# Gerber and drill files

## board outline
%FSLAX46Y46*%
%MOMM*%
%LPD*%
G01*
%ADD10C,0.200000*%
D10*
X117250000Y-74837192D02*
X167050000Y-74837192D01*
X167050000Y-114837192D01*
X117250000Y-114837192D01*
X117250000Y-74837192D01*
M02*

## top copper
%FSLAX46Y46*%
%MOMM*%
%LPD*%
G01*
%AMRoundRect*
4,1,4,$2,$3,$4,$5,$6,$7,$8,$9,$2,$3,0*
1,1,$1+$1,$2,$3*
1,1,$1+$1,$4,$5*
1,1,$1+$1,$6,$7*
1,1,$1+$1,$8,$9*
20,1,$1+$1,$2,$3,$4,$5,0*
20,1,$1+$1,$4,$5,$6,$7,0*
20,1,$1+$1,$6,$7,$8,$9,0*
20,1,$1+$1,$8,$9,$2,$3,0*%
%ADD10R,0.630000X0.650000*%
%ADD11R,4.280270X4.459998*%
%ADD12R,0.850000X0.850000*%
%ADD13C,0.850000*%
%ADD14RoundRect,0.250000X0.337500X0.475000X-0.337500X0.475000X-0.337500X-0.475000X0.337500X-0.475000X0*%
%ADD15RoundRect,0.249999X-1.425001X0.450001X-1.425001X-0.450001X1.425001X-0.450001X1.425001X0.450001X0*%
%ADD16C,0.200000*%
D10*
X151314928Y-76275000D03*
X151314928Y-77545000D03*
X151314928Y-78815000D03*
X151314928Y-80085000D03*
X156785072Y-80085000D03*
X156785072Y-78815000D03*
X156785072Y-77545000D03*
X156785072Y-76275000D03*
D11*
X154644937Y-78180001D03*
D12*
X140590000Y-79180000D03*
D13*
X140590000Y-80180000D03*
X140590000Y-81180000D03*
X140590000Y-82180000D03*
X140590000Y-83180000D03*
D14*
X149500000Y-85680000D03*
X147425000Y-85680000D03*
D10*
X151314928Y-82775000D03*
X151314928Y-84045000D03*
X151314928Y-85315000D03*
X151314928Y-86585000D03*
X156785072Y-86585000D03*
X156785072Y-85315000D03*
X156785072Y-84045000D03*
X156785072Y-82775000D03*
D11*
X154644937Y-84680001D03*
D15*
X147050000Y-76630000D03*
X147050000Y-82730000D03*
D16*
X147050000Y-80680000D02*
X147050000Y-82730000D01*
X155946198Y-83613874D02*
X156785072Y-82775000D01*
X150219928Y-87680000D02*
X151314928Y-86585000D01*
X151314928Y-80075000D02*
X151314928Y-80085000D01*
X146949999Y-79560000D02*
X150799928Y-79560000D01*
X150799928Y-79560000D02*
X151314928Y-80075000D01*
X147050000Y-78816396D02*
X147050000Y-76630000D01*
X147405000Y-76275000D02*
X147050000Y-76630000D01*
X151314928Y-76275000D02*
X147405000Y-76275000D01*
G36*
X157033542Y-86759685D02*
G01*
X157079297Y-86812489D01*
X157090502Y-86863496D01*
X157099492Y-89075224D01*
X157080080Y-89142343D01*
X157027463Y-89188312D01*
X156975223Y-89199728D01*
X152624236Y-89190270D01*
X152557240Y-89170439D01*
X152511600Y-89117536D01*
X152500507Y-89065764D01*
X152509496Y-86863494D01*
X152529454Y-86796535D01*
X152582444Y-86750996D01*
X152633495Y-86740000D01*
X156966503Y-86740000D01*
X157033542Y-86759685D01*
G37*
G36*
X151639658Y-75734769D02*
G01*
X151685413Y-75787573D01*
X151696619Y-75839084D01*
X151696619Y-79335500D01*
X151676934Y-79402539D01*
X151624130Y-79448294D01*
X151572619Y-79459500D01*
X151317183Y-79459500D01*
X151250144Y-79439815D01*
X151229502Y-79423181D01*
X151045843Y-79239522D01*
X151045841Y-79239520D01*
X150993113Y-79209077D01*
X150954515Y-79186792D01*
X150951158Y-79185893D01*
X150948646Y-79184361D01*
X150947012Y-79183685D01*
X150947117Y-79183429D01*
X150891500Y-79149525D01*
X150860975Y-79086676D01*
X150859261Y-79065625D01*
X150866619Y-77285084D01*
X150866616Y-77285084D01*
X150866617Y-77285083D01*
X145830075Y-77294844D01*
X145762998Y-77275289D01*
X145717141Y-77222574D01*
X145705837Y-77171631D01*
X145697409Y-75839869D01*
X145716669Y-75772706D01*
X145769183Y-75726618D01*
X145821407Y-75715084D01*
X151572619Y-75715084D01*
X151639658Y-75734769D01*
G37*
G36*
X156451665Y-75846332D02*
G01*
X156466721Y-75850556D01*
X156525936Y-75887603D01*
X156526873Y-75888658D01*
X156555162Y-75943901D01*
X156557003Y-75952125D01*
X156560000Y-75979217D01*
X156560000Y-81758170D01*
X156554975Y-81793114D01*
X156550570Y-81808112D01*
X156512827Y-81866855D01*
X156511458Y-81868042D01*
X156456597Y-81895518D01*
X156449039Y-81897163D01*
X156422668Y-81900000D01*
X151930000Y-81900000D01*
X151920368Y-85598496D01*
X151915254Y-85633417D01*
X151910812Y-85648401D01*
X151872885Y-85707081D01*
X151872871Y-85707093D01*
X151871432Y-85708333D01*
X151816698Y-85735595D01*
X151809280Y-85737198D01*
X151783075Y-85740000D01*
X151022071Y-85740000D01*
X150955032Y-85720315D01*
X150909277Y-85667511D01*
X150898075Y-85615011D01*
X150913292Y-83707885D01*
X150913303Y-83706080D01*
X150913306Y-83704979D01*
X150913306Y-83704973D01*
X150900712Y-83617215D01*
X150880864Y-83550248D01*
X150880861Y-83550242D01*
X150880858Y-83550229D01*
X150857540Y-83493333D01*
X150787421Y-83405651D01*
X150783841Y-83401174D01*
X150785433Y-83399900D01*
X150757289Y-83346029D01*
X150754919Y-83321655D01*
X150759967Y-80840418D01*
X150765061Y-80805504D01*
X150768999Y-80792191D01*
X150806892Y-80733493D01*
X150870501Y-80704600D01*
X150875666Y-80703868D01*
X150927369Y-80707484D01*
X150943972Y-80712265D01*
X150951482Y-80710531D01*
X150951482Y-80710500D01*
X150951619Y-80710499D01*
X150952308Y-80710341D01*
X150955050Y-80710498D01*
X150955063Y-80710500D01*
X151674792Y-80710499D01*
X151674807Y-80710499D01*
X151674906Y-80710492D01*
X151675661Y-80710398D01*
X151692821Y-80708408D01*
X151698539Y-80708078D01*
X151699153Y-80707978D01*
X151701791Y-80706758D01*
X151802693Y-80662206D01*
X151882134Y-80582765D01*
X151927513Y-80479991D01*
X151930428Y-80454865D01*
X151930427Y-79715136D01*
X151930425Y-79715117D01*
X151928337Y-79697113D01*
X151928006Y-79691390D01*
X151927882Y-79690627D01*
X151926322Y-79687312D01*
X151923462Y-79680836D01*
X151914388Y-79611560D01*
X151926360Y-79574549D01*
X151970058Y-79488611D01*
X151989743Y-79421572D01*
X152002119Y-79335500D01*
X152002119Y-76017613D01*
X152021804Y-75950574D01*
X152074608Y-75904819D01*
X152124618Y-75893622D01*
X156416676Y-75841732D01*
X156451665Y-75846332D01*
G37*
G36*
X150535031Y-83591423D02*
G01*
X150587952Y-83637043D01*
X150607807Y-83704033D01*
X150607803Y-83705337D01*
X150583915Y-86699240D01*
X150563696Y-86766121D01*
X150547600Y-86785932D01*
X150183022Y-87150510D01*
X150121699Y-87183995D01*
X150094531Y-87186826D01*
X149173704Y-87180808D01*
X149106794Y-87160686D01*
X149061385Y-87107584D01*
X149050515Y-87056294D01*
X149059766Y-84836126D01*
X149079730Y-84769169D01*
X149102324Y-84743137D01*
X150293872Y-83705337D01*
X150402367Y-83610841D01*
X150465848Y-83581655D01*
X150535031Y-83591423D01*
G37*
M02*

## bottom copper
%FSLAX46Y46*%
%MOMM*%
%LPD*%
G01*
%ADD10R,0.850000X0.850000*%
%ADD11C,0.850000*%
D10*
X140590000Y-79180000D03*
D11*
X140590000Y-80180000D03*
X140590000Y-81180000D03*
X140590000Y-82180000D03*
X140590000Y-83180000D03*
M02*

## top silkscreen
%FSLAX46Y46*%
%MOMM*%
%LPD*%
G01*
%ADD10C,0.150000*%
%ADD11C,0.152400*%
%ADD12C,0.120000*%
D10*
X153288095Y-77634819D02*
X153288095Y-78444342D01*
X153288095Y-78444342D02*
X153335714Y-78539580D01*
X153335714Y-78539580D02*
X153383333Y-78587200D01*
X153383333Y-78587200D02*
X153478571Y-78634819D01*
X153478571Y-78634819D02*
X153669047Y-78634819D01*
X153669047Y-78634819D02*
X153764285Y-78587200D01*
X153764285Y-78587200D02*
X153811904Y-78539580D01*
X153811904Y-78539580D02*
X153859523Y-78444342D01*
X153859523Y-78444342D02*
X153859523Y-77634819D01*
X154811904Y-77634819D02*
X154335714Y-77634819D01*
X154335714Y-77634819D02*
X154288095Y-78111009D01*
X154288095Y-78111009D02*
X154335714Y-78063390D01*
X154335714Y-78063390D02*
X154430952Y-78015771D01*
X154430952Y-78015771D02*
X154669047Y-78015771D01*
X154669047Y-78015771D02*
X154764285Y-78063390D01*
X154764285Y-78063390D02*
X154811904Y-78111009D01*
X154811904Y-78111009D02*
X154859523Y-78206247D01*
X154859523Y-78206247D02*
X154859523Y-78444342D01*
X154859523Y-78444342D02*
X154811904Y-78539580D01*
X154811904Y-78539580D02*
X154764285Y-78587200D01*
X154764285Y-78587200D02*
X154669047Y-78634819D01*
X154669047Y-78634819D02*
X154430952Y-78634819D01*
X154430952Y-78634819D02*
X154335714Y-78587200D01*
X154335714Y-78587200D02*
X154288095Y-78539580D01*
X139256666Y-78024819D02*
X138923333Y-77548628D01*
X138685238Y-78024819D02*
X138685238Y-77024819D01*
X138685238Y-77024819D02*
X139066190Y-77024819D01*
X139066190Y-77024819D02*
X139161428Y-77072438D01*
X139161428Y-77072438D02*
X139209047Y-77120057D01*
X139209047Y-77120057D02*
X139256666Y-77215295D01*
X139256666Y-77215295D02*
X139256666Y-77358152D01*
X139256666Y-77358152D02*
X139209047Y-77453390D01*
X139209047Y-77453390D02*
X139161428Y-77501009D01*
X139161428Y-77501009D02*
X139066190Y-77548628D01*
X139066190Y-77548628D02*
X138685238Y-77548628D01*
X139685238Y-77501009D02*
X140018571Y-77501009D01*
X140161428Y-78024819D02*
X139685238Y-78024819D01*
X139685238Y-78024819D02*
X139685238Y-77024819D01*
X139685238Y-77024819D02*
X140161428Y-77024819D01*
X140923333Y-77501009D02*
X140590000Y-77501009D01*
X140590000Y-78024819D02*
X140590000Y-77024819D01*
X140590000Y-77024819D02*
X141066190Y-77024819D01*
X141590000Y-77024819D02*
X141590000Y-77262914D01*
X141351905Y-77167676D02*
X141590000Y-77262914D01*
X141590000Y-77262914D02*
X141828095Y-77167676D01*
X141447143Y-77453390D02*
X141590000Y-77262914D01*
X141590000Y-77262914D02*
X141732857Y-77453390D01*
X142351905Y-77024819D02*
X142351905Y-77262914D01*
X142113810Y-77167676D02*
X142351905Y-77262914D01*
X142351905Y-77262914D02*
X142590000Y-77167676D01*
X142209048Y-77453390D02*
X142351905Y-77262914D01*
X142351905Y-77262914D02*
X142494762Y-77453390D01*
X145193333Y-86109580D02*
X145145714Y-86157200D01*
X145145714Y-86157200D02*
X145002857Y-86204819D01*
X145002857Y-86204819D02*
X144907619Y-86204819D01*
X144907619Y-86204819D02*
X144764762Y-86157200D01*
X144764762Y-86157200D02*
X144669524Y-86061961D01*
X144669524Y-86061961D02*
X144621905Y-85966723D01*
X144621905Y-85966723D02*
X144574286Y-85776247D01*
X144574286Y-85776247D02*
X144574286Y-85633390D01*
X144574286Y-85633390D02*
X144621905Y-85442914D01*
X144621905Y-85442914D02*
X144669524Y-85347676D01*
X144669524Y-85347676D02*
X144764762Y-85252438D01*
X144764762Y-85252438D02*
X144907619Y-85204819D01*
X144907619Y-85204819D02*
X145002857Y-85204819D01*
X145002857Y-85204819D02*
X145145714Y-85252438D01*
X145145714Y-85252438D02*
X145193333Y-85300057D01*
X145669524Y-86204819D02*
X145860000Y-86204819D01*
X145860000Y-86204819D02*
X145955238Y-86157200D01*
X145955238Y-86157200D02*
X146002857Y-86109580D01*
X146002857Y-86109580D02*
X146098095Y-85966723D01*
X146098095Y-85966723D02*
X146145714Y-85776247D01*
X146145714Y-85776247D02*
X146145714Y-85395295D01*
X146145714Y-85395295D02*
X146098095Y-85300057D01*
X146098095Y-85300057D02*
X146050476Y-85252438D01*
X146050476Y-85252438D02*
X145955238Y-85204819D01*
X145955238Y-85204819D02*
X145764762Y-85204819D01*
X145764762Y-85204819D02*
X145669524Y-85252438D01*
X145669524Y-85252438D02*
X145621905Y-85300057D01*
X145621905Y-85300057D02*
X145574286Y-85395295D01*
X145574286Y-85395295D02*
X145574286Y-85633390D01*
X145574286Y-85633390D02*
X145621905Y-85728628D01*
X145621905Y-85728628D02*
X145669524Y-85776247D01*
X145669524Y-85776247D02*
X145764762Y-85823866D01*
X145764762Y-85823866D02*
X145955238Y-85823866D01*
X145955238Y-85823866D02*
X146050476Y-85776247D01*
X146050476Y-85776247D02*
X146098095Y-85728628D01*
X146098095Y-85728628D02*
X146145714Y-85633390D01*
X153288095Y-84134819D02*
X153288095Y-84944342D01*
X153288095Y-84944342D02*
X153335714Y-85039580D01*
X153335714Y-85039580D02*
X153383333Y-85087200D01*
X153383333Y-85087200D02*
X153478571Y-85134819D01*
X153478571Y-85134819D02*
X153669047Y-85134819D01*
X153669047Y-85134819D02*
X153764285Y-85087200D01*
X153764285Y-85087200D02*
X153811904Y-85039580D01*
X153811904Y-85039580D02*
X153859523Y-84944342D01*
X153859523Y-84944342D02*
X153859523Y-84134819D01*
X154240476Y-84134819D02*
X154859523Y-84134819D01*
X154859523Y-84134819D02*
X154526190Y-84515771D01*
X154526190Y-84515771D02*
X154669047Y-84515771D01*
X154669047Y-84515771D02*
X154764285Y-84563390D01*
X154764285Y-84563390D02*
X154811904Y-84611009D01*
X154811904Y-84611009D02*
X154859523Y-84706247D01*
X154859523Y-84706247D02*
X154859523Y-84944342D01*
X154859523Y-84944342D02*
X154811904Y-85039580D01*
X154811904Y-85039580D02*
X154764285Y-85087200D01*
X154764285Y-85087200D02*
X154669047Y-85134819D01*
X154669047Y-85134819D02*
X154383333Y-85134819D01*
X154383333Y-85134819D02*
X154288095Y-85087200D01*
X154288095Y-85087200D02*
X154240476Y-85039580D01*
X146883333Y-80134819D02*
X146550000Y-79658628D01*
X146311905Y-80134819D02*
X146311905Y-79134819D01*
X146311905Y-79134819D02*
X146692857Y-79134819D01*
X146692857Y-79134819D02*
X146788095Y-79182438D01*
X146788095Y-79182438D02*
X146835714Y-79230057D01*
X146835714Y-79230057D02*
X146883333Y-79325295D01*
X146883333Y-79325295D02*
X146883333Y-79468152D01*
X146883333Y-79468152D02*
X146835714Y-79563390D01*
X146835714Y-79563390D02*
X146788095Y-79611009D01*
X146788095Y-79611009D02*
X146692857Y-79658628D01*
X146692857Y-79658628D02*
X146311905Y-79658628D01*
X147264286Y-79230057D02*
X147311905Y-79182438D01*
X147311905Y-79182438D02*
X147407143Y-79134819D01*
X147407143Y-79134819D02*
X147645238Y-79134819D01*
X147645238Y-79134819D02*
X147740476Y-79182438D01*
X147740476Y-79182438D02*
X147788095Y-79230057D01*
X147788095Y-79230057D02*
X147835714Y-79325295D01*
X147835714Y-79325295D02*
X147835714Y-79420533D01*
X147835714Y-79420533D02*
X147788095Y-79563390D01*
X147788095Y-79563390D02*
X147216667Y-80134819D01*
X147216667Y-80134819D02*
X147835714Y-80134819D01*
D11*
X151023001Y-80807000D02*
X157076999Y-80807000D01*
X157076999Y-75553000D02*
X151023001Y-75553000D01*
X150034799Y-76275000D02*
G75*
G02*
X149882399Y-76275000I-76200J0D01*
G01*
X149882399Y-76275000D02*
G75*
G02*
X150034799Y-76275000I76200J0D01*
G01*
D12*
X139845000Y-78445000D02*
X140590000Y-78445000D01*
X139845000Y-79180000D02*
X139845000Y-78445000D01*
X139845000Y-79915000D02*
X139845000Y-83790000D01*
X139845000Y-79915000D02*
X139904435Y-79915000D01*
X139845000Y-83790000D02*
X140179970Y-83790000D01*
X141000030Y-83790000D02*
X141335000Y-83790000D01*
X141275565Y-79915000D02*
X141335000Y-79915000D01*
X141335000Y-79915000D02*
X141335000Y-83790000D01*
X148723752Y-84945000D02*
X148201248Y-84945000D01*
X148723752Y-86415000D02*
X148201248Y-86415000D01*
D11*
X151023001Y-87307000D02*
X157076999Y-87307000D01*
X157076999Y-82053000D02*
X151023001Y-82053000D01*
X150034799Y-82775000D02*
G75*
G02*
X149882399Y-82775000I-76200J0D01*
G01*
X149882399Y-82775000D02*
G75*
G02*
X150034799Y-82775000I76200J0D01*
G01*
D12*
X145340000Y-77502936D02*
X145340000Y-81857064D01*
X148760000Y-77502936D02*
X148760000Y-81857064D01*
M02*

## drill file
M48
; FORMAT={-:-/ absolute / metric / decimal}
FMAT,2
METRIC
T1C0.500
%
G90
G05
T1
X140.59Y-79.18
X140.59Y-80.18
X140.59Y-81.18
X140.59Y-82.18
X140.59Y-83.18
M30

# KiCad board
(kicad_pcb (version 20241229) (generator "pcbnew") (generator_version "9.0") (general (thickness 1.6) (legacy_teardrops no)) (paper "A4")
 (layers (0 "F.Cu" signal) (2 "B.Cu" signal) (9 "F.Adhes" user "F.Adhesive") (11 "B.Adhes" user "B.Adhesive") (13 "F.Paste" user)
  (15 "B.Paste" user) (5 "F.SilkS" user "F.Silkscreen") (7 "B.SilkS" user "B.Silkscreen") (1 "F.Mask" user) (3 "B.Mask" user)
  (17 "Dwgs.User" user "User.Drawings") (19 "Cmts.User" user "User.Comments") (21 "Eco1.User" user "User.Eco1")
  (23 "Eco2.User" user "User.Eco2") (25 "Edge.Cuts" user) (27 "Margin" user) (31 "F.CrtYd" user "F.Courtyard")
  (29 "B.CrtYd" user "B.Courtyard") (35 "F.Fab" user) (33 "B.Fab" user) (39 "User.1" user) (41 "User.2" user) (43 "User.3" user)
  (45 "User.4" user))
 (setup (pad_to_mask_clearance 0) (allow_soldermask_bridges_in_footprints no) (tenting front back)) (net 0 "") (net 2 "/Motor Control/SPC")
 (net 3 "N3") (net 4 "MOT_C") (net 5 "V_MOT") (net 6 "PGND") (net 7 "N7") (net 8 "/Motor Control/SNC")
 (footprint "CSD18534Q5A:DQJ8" (layer "F.Cu") (at 154.05 78.18)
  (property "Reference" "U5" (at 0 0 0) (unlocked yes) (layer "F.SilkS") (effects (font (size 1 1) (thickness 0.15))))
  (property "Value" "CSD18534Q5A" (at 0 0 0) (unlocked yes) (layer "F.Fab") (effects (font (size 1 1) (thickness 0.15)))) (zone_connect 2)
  (fp_line (start -3.026999 2.627) (end 3.026999 2.627) (stroke (width 0.1524) (type solid)) (layer "F.SilkS") (net 1))
  (fp_line (start 3.026999 -2.627) (end -3.026999 -2.627) (stroke (width 0.1524) (type solid)) (layer "F.SilkS") (net 1))
  (fp_circle (center -4.091401 -1.905) (end -4.015201 -1.905) (stroke (width 0.1524) (type solid)) (fill no) (layer "F.SilkS") (net 1))
  (pad "1" smd rect (at -2.735072 -1.905) (size 0.63 0.65) (layers "F.Cu" "F.Mask" "F.Paste") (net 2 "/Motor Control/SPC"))
  (pad "2" smd rect (at -2.735072 -0.635) (size 0.63 0.65) (layers "F.Cu" "F.Mask" "F.Paste") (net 2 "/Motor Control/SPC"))
  (pad "3" smd rect (at -2.735072 0.635) (size 0.63 0.65) (layers "F.Cu" "F.Mask" "F.Paste") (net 2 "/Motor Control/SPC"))
  (pad "4" smd rect (at -2.735072 1.905) (size 0.63 0.65) (layers "F.Cu" "F.Mask" "F.Paste") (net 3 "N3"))
  (pad "5" smd rect (at 2.735072 1.905) (size 0.63 0.65) (layers "F.Cu" "F.Mask" "F.Paste") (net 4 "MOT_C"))
  (pad "6" smd rect (at 2.735072 0.635) (size 0.63 0.65) (layers "F.Cu" "F.Mask" "F.Paste") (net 4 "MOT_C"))
  (pad "7" smd rect (at 2.735072 -0.635) (size 0.63 0.65) (layers "F.Cu" "F.Mask" "F.Paste") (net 4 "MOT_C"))
  (pad "8" smd rect (at 2.735072 -1.905) (size 0.63 0.65) (layers "F.Cu" "F.Mask" "F.Paste") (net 4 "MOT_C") (clearance 0) (zone_connect 2)
   (thermal_bridge_width 0.25) (thermal_gap 0.25))
  (pad "9" smd rect (at 0.594937 0.000001) (size 4.28027 4.459998) (layers "F.Cu" "F.Mask" "F.Paste") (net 4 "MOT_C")))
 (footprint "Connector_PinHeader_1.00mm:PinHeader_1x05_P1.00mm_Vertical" (layer "F.Cu") (at 140.59 79.18)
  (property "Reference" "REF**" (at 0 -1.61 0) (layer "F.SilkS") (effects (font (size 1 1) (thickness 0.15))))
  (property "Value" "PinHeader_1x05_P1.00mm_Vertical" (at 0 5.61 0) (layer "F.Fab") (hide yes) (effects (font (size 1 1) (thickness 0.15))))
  (fp_line (start -0.745 -0.735) (end 0 -0.735) (stroke (width 0.12) (type solid)) (layer "F.SilkS"))
  (fp_line (start -0.745 0) (end -0.745 -0.735) (stroke (width 0.12) (type solid)) (layer "F.SilkS"))
  (fp_line (start -0.745 0.735) (end -0.745 4.61) (stroke (width 0.12) (type solid)) (layer "F.SilkS"))
  (fp_line (start -0.745 0.735) (end -0.685565 0.735) (stroke (width 0.12) (type solid)) (layer "F.SilkS"))
  (fp_line (start -0.745 4.61) (end -0.41003 4.61) (stroke (width 0.12) (type solid)) (layer "F.SilkS"))
  (fp_line (start 0.41003 4.61) (end 0.745 4.61) (stroke (width 0.12) (type solid)) (layer "F.SilkS"))
  (fp_line (start 0.685565 0.735) (end 0.745 0.735) (stroke (width 0.12) (type solid)) (layer "F.SilkS"))
  (fp_line (start 0.745 0.735) (end 0.745 4.61) (stroke (width 0.12) (type solid)) (layer "F.SilkS"))
  (pad "1" thru_hole rect (at 0 0) (size 0.85 0.85) (drill 0.5) (layers "*.Cu" "*.Mask") (remove_unused_layers no))
  (pad "2" thru_hole circle (at 0 1) (size 0.85 0.85) (drill 0.5) (layers "*.Cu" "*.Mask") (remove_unused_layers no))
  (pad "3" thru_hole circle (at 0 2) (size 0.85 0.85) (drill 0.5) (layers "*.Cu" "*.Mask") (remove_unused_layers no))
  (pad "4" thru_hole circle (at 0 3) (size 0.85 0.85) (drill 0.5) (layers "*.Cu" "*.Mask") (remove_unused_layers no))
  (pad "5" thru_hole circle (at 0 4) (size 0.85 0.85) (drill 0.5) (layers "*.Cu" "*.Mask") (remove_unused_layers no)))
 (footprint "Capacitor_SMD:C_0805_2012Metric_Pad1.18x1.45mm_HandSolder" (layer "F.Cu") (at 148.4625 85.68 180)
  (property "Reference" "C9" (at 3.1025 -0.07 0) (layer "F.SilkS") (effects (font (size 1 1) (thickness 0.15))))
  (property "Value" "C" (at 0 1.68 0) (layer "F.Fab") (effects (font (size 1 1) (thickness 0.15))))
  (fp_line (start -0.261252 0.735) (end 0.261252 0.735) (stroke (width 0.12) (type solid)) (layer "F.SilkS") (net 1))
  (fp_line (start -0.261252 -0.735) (end 0.261252 -0.735) (stroke (width 0.12) (type solid)) (layer "F.SilkS") (net 1))
  (pad "1" smd roundrect (at -1.0375 0 180) (size 1.175 1.45) (layers "F.Cu" "F.Mask" "F.Paste") (roundrect_rratio 0.212766) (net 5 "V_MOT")
   (zone_connect 2))
  (pad "2" smd roundrect (at 1.0375 0 180) (size 1.175 1.45) (layers "F.Cu" "F.Mask" "F.Paste") (roundrect_rratio 0.212766) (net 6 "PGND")))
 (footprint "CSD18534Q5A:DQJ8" (layer "F.Cu") (at 154.05 84.68)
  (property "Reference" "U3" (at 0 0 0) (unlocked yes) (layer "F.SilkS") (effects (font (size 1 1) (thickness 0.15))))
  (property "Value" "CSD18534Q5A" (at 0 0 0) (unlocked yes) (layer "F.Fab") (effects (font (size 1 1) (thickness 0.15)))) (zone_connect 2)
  (fp_line (start -3.026999 2.627) (end 3.026999 2.627) (stroke (width 0.1524) (type solid)) (layer "F.SilkS") (net 1))
  (fp_line (start 3.026999 -2.627) (end -3.026999 -2.627) (stroke (width 0.1524) (type solid)) (layer "F.SilkS") (net 1))
  (fp_circle (center -4.091401 -1.905) (end -4.015201 -1.905) (stroke (width 0.1524) (type solid)) (fill no) (layer "F.SilkS") (net 1))
  (pad "1" smd rect (at -2.735072 -1.905) (size 0.63 0.65) (layers "F.Cu" "F.Mask" "F.Paste") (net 4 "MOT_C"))
  (pad "2" smd rect (at -2.735072 -0.635) (size 0.63 0.65) (layers "F.Cu" "F.Mask" "F.Paste") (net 4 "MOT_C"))
  (pad "3" smd rect (at -2.735072 0.635) (size 0.63 0.65) (layers "F.Cu" "F.Mask" "F.Paste") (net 4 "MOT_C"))
  (pad "4" smd rect (at -2.735072 1.905) (size 0.63 0.65) (layers "F.Cu" "F.Mask" "F.Paste") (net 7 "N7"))
  (pad "5" smd rect (at 2.735072 1.905) (size 0.63 0.65) (layers "F.Cu" "F.Mask" "F.Paste") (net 5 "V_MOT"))
  (pad "6" smd rect (at 2.735072 0.635) (size 0.63 0.65) (layers "F.Cu" "F.Mask" "F.Paste") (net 5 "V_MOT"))
  (pad "7" smd rect (at 2.735072 -0.635) (size 0.63 0.65) (layers "F.Cu" "F.Mask" "F.Paste") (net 5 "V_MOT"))
  (pad "8" smd rect (at 2.735072 -1.905) (size 0.63 0.65) (layers "F.Cu" "F.Mask" "F.Paste") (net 5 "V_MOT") (clearance 0) (zone_connect 2)
   (thermal_bridge_width 0.25) (thermal_gap 0.25))
  (pad "9" smd rect (at 0.594937 0.000001) (size 4.28027 4.459998) (layers "F.Cu" "F.Mask" "F.Paste") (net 5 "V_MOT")))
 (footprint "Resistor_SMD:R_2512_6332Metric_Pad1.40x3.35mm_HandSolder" (layer "F.Cu") (at 147.05 79.68 -90)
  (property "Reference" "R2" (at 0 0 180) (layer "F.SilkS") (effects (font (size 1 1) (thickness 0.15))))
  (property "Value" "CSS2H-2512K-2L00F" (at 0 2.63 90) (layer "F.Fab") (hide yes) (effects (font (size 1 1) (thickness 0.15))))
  (fp_line (start -2.177064 1.71) (end 2.177064 1.71) (stroke (width 0.12) (type solid)) (layer "F.SilkS") (net 1))
  (fp_line (start -2.177064 -1.71) (end 2.177064 -1.71) (stroke (width 0.12) (type solid)) (layer "F.SilkS") (net 1))
  (pad "1" smd roundrect (at -3.05 0 270) (size 1.4 3.35) (layers "F.Cu" "F.Mask" "F.Paste") (roundrect_rratio 0.178571)
   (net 2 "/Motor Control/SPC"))
  (pad "2" smd roundrect (at 3.05 0 270) (size 1.4 3.35) (layers "F.Cu" "F.Mask" "F.Paste") (roundrect_rratio 0.178571)
   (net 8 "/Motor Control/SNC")))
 (gr_rect (start 117.25 74.837192) (end 167.05 114.837192) (stroke (width 0.2) (type default)) (fill no) (layer "Edge.Cuts"))
 (segment (start 147.05 80.68) (end 147.05 82.73) (width 0.2) (layer "F.Cu") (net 8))
 (segment (start 155.946198 83.613874) (end 156.785072 82.775) (width 0.2) (layer "F.Cu") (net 5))
 (segment (start 150.219928 87.68) (end 151.314928 86.585) (width 0.2) (layer "F.Cu") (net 7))
 (segment (start 151.314928 80.075) (end 151.314928 80.085) (width 0.2) (layer "F.Cu") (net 3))
 (segment (start 146.949999 79.56) (end 150.799928 79.56) (width 0.2) (layer "F.Cu") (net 3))
 (segment (start 150.799928 79.56) (end 151.314928 80.075) (width 0.2) (layer "F.Cu") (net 3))
 (segment (start 147.05 78.816396) (end 147.05 76.63) (width 0.2) (layer "F.Cu") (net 2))
 (segment (start 147.405 76.275) (end 147.05 76.63) (width 0.2) (layer "F.Cu") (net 2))
 (segment (start 151.314928 76.275) (end 147.405 76.275) (width 0.2) (layer "F.Cu") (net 2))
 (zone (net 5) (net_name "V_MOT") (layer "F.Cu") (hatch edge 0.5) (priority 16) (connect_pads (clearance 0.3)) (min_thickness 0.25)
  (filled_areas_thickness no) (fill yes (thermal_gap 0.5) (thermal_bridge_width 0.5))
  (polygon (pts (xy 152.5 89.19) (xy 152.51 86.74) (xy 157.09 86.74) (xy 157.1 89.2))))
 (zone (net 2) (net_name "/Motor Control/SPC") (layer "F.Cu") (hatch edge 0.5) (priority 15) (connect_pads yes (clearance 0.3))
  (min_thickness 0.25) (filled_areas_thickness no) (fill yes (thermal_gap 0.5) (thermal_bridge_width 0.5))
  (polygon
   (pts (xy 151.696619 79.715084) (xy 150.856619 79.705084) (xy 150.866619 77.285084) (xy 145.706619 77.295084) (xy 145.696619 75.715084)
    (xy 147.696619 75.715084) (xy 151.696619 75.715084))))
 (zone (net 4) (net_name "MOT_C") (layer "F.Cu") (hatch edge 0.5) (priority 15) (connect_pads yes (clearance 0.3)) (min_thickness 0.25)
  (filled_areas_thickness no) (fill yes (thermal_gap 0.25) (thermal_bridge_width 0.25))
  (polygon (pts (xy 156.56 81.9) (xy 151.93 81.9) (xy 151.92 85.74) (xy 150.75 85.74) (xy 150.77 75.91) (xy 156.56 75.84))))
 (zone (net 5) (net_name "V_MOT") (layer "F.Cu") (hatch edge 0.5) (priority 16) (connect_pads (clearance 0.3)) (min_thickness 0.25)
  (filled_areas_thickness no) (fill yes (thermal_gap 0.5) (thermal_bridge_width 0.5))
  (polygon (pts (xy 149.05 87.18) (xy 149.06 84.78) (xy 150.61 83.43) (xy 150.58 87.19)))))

